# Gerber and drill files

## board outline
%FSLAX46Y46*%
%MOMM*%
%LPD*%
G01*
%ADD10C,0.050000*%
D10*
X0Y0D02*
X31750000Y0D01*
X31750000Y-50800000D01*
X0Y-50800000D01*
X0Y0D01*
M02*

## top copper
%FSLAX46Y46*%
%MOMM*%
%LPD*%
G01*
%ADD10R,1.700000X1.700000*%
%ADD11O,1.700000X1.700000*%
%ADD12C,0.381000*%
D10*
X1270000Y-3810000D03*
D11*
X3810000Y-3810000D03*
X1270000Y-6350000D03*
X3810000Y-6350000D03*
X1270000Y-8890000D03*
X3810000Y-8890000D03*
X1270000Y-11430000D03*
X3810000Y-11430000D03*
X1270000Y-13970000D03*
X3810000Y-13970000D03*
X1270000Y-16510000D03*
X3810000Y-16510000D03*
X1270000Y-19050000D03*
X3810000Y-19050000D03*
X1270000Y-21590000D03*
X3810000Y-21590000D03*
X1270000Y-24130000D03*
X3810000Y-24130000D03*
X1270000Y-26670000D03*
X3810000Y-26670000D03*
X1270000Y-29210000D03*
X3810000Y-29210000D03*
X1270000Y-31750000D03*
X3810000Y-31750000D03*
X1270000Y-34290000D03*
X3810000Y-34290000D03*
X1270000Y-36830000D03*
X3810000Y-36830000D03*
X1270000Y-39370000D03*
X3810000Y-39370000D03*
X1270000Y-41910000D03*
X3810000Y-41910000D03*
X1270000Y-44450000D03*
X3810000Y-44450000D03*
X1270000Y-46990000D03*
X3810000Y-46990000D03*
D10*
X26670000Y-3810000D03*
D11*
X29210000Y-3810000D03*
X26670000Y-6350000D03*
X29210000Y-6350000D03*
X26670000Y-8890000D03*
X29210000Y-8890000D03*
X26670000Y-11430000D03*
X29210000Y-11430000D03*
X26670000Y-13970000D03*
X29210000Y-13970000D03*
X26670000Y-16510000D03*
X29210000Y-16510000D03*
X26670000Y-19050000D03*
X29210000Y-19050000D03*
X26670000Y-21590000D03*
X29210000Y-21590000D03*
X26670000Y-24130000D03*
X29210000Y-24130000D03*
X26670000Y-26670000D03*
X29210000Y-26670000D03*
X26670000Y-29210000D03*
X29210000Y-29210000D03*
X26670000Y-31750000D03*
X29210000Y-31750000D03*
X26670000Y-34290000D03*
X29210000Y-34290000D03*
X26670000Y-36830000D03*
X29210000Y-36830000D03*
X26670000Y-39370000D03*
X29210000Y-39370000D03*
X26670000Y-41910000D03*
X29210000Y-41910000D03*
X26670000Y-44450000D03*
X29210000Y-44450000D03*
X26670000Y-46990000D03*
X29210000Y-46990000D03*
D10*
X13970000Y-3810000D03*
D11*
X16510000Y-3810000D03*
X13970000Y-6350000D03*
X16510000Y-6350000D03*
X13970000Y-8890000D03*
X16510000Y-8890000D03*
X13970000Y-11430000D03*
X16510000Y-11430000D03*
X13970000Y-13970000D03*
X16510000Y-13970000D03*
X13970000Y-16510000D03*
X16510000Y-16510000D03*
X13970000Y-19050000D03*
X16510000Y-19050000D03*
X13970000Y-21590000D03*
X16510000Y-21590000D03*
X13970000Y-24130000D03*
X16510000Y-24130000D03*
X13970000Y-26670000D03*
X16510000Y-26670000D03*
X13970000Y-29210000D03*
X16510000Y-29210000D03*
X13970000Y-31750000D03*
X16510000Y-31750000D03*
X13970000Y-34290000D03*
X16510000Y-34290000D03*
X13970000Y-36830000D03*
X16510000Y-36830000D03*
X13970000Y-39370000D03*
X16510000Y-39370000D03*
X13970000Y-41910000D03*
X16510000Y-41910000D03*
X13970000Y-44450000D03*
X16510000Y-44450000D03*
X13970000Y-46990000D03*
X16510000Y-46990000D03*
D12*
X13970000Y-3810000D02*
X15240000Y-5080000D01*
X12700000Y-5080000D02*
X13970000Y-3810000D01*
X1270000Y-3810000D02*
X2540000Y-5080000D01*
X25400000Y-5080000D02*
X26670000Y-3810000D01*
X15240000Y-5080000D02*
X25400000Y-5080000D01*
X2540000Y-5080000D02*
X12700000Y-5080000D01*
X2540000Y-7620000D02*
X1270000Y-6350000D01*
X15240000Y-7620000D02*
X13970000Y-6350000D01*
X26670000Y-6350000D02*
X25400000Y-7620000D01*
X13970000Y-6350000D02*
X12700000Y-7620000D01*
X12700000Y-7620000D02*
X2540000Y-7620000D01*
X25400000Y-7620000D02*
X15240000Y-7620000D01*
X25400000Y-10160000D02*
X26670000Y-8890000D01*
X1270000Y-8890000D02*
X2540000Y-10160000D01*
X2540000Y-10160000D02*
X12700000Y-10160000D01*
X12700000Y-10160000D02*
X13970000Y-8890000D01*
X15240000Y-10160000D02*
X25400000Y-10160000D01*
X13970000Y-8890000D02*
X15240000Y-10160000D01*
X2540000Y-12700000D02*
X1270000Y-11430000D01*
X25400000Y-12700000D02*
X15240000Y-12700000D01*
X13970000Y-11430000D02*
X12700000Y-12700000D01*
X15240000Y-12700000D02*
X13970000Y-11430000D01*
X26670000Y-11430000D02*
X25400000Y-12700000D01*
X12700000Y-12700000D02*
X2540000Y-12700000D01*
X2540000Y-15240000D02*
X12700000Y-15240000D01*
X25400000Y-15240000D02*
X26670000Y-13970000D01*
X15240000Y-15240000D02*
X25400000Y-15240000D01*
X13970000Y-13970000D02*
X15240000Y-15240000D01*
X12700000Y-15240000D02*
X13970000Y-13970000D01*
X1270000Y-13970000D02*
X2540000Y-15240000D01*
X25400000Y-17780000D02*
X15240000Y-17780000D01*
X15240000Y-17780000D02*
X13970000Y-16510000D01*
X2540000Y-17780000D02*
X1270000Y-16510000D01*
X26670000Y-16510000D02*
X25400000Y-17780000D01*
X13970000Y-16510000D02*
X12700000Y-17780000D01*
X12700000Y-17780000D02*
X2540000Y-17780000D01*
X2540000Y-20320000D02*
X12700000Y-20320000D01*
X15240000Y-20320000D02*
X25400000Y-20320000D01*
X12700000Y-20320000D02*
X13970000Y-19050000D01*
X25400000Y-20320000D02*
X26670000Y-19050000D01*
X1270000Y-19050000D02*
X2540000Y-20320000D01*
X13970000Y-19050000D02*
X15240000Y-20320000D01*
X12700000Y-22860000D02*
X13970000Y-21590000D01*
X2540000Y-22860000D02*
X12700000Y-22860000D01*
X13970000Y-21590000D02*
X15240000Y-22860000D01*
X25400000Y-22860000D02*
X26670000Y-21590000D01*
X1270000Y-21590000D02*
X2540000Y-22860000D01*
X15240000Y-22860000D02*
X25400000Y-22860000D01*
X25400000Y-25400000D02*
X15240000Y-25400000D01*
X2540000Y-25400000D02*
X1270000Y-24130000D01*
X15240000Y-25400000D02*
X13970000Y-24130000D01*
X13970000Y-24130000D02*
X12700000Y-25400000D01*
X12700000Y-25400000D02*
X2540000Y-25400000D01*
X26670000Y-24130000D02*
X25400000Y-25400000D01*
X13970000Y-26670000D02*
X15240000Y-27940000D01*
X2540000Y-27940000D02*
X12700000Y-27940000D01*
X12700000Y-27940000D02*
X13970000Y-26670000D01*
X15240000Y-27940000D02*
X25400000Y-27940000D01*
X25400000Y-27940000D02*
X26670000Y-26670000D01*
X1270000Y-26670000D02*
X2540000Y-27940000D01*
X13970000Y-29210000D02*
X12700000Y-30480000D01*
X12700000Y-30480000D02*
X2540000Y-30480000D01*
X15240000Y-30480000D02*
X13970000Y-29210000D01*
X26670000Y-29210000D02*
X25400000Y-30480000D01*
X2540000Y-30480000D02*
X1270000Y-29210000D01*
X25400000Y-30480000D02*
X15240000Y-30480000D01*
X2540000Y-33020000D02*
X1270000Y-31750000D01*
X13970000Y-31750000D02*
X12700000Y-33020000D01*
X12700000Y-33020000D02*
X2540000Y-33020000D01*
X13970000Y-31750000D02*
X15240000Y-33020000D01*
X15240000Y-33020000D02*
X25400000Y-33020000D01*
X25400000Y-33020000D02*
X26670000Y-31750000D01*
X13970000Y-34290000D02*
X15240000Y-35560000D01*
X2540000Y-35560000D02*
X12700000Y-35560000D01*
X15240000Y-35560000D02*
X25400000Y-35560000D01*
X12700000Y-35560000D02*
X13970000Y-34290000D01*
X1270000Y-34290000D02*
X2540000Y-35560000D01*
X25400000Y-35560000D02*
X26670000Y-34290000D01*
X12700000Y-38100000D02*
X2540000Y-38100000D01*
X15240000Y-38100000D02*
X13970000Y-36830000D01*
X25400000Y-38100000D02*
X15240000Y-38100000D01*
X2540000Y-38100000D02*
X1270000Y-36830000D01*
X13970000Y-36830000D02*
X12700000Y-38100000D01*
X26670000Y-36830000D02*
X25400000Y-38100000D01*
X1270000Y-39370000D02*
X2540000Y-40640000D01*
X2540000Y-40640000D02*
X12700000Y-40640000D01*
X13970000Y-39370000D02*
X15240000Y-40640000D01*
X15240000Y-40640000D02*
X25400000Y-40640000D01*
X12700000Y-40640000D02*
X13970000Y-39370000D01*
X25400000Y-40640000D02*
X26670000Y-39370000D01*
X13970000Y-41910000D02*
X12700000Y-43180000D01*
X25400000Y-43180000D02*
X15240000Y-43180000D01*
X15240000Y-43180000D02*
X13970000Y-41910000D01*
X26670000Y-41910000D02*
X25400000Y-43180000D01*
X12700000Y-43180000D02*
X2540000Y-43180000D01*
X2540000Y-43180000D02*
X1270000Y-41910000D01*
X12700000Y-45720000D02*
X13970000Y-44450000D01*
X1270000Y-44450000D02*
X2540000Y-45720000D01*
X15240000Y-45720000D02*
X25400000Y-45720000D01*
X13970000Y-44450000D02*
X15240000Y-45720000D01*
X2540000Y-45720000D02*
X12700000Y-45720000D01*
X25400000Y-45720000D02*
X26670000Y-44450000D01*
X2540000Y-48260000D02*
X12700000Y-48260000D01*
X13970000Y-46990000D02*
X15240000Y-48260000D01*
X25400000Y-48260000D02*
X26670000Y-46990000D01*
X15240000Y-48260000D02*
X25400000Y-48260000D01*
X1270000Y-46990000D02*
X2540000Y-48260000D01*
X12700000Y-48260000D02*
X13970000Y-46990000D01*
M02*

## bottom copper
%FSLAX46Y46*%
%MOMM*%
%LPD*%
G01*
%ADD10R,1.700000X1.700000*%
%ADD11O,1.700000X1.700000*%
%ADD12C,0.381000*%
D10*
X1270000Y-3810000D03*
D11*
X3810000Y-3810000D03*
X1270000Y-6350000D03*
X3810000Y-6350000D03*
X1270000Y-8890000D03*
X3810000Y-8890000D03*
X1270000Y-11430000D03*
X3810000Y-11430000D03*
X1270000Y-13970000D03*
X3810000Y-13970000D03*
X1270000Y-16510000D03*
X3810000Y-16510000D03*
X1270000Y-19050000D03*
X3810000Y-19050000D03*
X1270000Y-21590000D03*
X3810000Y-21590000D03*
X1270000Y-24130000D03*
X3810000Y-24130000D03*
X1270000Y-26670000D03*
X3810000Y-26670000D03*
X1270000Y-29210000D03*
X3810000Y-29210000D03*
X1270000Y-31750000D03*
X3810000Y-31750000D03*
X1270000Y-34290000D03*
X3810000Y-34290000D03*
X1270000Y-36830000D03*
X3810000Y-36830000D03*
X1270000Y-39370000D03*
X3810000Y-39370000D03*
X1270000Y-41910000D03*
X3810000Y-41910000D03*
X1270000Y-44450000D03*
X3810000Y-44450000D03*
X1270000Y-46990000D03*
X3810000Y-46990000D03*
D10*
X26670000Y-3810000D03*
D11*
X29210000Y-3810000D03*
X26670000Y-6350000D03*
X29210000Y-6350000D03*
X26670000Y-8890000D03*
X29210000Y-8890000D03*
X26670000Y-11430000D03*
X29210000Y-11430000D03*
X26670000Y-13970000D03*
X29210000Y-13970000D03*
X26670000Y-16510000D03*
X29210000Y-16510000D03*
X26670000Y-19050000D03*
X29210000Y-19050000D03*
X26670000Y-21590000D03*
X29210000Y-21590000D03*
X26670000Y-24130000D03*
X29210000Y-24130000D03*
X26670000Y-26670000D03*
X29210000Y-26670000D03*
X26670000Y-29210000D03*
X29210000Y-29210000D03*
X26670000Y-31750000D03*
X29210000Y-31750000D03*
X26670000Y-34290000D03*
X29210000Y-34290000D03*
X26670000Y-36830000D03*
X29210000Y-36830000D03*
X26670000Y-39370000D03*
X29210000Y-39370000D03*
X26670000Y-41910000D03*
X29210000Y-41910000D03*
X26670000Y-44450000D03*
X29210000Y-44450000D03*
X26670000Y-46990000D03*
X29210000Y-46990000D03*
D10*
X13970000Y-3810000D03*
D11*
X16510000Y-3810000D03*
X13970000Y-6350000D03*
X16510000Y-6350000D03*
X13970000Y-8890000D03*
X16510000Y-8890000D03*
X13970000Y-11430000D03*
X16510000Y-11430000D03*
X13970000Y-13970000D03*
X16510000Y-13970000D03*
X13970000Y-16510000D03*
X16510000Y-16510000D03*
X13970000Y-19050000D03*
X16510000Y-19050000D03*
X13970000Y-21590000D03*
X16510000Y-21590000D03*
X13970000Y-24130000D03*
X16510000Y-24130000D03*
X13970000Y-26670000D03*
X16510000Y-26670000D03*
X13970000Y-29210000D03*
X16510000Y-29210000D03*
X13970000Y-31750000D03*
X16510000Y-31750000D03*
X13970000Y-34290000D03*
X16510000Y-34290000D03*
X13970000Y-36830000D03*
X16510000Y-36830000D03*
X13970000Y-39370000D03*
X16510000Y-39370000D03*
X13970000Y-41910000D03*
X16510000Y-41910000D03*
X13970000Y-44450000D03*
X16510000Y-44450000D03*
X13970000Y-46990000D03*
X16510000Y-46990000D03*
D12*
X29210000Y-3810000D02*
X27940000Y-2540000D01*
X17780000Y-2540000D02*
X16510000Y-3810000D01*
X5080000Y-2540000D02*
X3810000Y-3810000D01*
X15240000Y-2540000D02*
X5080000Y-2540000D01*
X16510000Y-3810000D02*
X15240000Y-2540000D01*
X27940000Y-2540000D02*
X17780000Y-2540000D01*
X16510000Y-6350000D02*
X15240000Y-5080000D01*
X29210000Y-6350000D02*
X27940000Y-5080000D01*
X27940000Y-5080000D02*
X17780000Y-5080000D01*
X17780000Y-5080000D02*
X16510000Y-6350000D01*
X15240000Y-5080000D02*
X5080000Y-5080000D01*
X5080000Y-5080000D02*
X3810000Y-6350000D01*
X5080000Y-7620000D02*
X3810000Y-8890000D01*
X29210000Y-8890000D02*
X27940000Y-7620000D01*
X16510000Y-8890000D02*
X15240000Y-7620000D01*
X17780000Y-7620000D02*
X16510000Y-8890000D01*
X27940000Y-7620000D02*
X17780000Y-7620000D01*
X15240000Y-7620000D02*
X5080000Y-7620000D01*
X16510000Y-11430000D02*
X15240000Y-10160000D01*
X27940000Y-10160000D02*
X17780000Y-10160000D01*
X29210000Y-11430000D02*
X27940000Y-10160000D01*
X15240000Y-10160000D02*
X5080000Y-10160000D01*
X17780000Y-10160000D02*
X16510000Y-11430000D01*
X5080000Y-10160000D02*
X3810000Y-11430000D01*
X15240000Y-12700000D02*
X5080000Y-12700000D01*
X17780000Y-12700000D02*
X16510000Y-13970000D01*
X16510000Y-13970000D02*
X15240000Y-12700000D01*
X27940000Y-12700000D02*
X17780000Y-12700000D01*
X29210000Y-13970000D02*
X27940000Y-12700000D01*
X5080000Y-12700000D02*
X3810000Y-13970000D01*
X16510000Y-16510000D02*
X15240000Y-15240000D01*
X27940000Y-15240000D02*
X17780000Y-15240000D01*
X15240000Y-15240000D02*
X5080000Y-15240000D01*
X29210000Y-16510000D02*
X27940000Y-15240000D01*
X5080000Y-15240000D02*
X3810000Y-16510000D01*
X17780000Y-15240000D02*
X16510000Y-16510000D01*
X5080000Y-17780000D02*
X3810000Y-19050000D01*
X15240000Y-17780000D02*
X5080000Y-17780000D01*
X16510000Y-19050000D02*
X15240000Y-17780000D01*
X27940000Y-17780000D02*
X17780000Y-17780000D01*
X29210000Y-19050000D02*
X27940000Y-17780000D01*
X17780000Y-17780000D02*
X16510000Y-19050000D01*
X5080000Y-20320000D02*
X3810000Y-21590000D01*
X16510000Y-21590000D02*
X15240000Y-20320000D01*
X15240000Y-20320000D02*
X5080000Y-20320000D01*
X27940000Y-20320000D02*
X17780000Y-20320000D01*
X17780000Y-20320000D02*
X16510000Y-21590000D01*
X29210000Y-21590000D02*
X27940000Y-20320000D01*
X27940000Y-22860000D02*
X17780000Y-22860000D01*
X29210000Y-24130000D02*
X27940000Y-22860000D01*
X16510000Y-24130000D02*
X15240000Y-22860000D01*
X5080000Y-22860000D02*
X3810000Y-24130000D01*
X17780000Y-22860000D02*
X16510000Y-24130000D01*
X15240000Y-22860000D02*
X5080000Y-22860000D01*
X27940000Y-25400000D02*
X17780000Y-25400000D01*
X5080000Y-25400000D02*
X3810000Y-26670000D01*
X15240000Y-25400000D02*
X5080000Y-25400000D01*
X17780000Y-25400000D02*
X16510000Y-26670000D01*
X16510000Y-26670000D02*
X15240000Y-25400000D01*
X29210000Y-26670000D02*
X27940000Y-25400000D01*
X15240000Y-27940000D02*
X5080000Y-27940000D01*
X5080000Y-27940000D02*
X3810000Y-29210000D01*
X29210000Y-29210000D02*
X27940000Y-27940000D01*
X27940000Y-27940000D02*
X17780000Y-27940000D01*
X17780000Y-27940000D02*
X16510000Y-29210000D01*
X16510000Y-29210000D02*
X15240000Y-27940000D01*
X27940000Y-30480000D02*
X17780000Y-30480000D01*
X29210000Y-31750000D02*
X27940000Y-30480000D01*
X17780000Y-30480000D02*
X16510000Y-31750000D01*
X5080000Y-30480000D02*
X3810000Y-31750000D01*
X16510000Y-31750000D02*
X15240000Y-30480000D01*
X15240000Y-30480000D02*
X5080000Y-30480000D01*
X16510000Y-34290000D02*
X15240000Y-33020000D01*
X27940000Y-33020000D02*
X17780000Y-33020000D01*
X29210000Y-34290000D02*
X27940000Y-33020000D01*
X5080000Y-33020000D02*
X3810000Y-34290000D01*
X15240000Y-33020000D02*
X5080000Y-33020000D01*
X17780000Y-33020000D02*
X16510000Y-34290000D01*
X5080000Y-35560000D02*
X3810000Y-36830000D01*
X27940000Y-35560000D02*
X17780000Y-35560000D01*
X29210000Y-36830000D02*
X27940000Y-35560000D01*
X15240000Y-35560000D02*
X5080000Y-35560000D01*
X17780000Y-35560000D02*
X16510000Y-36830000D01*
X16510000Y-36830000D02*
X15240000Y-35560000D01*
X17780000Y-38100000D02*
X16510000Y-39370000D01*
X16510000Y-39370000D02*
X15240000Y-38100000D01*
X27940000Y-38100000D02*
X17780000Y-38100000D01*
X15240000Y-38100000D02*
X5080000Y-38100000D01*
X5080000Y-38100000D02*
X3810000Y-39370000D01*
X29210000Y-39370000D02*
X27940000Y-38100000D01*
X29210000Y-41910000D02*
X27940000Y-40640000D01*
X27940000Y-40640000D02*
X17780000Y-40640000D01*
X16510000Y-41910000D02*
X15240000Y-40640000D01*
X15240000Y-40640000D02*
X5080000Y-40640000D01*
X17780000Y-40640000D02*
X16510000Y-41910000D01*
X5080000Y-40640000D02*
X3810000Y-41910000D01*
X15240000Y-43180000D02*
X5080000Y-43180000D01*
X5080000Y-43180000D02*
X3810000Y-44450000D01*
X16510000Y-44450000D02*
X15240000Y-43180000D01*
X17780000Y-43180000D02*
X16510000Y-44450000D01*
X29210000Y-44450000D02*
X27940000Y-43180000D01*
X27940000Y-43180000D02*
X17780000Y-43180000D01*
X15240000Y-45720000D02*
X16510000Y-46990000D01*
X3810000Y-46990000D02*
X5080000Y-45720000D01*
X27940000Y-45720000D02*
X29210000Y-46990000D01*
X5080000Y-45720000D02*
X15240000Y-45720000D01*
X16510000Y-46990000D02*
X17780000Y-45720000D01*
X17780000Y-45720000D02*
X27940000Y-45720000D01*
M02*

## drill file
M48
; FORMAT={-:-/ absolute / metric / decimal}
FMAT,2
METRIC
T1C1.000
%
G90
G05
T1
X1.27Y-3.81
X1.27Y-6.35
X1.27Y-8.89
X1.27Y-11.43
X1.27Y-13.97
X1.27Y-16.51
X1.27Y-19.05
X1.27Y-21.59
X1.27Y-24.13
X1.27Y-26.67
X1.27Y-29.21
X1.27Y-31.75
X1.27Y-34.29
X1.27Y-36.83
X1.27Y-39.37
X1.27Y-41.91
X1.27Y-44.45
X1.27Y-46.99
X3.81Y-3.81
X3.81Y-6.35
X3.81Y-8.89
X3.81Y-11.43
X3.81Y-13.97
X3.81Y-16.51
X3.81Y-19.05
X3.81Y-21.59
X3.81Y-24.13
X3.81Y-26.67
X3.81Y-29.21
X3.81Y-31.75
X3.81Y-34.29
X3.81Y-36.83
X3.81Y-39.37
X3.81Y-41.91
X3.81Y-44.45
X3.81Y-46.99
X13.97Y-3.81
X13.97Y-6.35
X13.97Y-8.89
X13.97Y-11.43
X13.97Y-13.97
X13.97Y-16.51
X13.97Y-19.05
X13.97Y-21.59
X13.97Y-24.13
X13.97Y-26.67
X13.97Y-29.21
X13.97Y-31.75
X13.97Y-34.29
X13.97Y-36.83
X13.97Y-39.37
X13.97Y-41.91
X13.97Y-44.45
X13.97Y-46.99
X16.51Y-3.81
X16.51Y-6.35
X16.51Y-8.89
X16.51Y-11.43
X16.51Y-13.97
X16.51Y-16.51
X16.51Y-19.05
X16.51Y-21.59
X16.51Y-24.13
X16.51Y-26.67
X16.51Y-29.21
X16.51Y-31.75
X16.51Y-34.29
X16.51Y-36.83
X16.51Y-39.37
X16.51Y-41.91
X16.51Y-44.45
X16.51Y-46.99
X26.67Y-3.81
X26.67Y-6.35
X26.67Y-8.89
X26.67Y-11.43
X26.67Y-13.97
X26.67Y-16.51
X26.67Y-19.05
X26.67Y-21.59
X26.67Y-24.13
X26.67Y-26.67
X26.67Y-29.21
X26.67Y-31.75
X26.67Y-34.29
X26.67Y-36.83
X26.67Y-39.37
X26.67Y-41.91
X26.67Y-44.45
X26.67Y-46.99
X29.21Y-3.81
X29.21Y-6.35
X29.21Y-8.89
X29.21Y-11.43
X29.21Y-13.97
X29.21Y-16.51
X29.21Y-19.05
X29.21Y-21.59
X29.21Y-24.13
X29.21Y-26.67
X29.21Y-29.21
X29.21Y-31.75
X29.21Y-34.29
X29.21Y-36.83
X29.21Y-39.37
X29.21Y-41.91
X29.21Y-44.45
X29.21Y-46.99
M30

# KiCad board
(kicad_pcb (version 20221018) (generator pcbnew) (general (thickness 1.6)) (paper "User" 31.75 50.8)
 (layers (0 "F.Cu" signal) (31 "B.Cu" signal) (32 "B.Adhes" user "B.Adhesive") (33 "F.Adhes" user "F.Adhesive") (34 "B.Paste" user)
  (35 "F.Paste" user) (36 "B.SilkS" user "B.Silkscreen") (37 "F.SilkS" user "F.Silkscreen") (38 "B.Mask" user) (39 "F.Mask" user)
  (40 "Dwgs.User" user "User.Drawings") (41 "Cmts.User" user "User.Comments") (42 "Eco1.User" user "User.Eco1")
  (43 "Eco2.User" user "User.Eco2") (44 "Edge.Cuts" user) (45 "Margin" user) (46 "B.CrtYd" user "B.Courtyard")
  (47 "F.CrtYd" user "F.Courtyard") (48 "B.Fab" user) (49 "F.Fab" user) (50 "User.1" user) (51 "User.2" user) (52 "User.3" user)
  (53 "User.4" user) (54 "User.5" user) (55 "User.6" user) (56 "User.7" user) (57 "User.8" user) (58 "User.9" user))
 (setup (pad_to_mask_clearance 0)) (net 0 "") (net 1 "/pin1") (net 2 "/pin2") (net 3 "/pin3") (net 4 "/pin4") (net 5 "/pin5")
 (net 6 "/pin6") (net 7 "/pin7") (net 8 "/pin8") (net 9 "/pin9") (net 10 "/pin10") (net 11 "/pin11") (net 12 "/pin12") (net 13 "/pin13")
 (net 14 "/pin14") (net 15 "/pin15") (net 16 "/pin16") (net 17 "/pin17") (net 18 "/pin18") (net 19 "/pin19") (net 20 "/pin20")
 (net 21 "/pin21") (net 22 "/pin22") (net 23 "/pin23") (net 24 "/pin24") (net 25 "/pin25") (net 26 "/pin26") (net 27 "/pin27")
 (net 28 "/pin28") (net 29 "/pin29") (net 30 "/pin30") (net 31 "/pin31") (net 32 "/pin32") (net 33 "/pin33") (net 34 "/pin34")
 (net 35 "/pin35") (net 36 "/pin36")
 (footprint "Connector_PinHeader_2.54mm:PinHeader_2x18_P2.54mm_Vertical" (layer "F.Cu") (at 1.27 3.81)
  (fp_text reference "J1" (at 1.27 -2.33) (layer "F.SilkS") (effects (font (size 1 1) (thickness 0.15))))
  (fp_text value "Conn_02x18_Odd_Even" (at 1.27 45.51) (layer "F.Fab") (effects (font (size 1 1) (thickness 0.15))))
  (pad "1" thru_hole rect (at 0 0) (size 1.7 1.7) (drill 1) (layers "*.Cu" "*.Mask") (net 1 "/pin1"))
  (pad "2" thru_hole oval (at 2.54 0) (size 1.7 1.7) (drill 1) (layers "*.Cu" "*.Mask") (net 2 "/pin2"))
  (pad "3" thru_hole oval (at 0 2.54) (size 1.7 1.7) (drill 1) (layers "*.Cu" "*.Mask") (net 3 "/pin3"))
  (pad "4" thru_hole oval (at 2.54 2.54) (size 1.7 1.7) (drill 1) (layers "*.Cu" "*.Mask") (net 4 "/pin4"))
  (pad "5" thru_hole oval (at 0 5.08) (size 1.7 1.7) (drill 1) (layers "*.Cu" "*.Mask") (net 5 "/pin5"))
  (pad "6" thru_hole oval (at 2.54 5.08) (size 1.7 1.7) (drill 1) (layers "*.Cu" "*.Mask") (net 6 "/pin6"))
  (pad "7" thru_hole oval (at 0 7.62) (size 1.7 1.7) (drill 1) (layers "*.Cu" "*.Mask") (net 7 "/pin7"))
  (pad "8" thru_hole oval (at 2.54 7.62) (size 1.7 1.7) (drill 1) (layers "*.Cu" "*.Mask") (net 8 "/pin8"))
  (pad "9" thru_hole oval (at 0 10.16) (size 1.7 1.7) (drill 1) (layers "*.Cu" "*.Mask") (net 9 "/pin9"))
  (pad "10" thru_hole oval (at 2.54 10.16) (size 1.7 1.7) (drill 1) (layers "*.Cu" "*.Mask") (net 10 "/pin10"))
  (pad "11" thru_hole oval (at 0 12.7) (size 1.7 1.7) (drill 1) (layers "*.Cu" "*.Mask") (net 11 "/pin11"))
  (pad "12" thru_hole oval (at 2.54 12.7) (size 1.7 1.7) (drill 1) (layers "*.Cu" "*.Mask") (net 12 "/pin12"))
  (pad "13" thru_hole oval (at 0 15.24) (size 1.7 1.7) (drill 1) (layers "*.Cu" "*.Mask") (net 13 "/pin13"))
  (pad "14" thru_hole oval (at 2.54 15.24) (size 1.7 1.7) (drill 1) (layers "*.Cu" "*.Mask") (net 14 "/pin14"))
  (pad "15" thru_hole oval (at 0 17.78) (size 1.7 1.7) (drill 1) (layers "*.Cu" "*.Mask") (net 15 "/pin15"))
  (pad "16" thru_hole oval (at 2.54 17.78) (size 1.7 1.7) (drill 1) (layers "*.Cu" "*.Mask") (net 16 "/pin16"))
  (pad "17" thru_hole oval (at 0 20.32) (size 1.7 1.7) (drill 1) (layers "*.Cu" "*.Mask") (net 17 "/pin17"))
  (pad "18" thru_hole oval (at 2.54 20.32) (size 1.7 1.7) (drill 1) (layers "*.Cu" "*.Mask") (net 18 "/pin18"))
  (pad "19" thru_hole oval (at 0 22.86) (size 1.7 1.7) (drill 1) (layers "*.Cu" "*.Mask") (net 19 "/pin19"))
  (pad "20" thru_hole oval (at 2.54 22.86) (size 1.7 1.7) (drill 1) (layers "*.Cu" "*.Mask") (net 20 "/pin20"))
  (pad "21" thru_hole oval (at 0 25.4) (size 1.7 1.7) (drill 1) (layers "*.Cu" "*.Mask") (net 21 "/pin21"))
  (pad "22" thru_hole oval (at 2.54 25.4) (size 1.7 1.7) (drill 1) (layers "*.Cu" "*.Mask") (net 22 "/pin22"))
  (pad "23" thru_hole oval (at 0 27.94) (size 1.7 1.7) (drill 1) (layers "*.Cu" "*.Mask") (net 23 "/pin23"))
  (pad "24" thru_hole oval (at 2.54 27.94) (size 1.7 1.7) (drill 1) (layers "*.Cu" "*.Mask") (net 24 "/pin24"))
  (pad "25" thru_hole oval (at 0 30.48) (size 1.7 1.7) (drill 1) (layers "*.Cu" "*.Mask") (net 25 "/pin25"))
  (pad "26" thru_hole oval (at 2.54 30.48) (size 1.7 1.7) (drill 1) (layers "*.Cu" "*.Mask") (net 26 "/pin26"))
  (pad "27" thru_hole oval (at 0 33.02) (size 1.7 1.7) (drill 1) (layers "*.Cu" "*.Mask") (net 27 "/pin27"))
  (pad "28" thru_hole oval (at 2.54 33.02) (size 1.7 1.7) (drill 1) (layers "*.Cu" "*.Mask") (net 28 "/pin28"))
  (pad "29" thru_hole oval (at 0 35.56) (size 1.7 1.7) (drill 1) (layers "*.Cu" "*.Mask") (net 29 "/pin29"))
  (pad "30" thru_hole oval (at 2.54 35.56) (size 1.7 1.7) (drill 1) (layers "*.Cu" "*.Mask") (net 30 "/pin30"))
  (pad "31" thru_hole oval (at 0 38.1) (size 1.7 1.7) (drill 1) (layers "*.Cu" "*.Mask") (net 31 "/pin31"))
  (pad "32" thru_hole oval (at 2.54 38.1) (size 1.7 1.7) (drill 1) (layers "*.Cu" "*.Mask") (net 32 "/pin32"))
  (pad "33" thru_hole oval (at 0 40.64) (size 1.7 1.7) (drill 1) (layers "*.Cu" "*.Mask") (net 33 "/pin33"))
  (pad "34" thru_hole oval (at 2.54 40.64) (size 1.7 1.7) (drill 1) (layers "*.Cu" "*.Mask") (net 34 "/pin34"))
  (pad "35" thru_hole oval (at 0 43.18) (size 1.7 1.7) (drill 1) (layers "*.Cu" "*.Mask") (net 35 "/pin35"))
  (pad "36" thru_hole oval (at 2.54 43.18) (size 1.7 1.7) (drill 1) (layers "*.Cu" "*.Mask") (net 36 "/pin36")))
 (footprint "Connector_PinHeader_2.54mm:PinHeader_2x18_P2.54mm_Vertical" (layer "F.Cu") (at 26.67 3.81)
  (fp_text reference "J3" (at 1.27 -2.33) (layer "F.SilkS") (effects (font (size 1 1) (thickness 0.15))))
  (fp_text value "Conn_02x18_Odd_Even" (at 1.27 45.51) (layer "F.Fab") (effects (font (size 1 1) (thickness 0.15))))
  (pad "1" thru_hole rect (at 0 0) (size 1.7 1.7) (drill 1) (layers "*.Cu" "*.Mask") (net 1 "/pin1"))
  (pad "2" thru_hole oval (at 2.54 0) (size 1.7 1.7) (drill 1) (layers "*.Cu" "*.Mask") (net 2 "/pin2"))
  (pad "3" thru_hole oval (at 0 2.54) (size 1.7 1.7) (drill 1) (layers "*.Cu" "*.Mask") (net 3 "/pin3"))
  (pad "4" thru_hole oval (at 2.54 2.54) (size 1.7 1.7) (drill 1) (layers "*.Cu" "*.Mask") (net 4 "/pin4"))
  (pad "5" thru_hole oval (at 0 5.08) (size 1.7 1.7) (drill 1) (layers "*.Cu" "*.Mask") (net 5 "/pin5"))
  (pad "6" thru_hole oval (at 2.54 5.08) (size 1.7 1.7) (drill 1) (layers "*.Cu" "*.Mask") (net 6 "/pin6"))
  (pad "7" thru_hole oval (at 0 7.62) (size 1.7 1.7) (drill 1) (layers "*.Cu" "*.Mask") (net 7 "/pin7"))
  (pad "8" thru_hole oval (at 2.54 7.62) (size 1.7 1.7) (drill 1) (layers "*.Cu" "*.Mask") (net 8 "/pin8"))
  (pad "9" thru_hole oval (at 0 10.16) (size 1.7 1.7) (drill 1) (layers "*.Cu" "*.Mask") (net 9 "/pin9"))
  (pad "10" thru_hole oval (at 2.54 10.16) (size 1.7 1.7) (drill 1) (layers "*.Cu" "*.Mask") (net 10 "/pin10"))
  (pad "11" thru_hole oval (at 0 12.7) (size 1.7 1.7) (drill 1) (layers "*.Cu" "*.Mask") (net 11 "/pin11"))
  (pad "12" thru_hole oval (at 2.54 12.7) (size 1.7 1.7) (drill 1) (layers "*.Cu" "*.Mask") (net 12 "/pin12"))
  (pad "13" thru_hole oval (at 0 15.24) (size 1.7 1.7) (drill 1) (layers "*.Cu" "*.Mask") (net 13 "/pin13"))
  (pad "14" thru_hole oval (at 2.54 15.24) (size 1.7 1.7) (drill 1) (layers "*.Cu" "*.Mask") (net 14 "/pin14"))
  (pad "15" thru_hole oval (at 0 17.78) (size 1.7 1.7) (drill 1) (layers "*.Cu" "*.Mask") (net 15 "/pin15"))
  (pad "16" thru_hole oval (at 2.54 17.78) (size 1.7 1.7) (drill 1) (layers "*.Cu" "*.Mask") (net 16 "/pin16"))
  (pad "17" thru_hole oval (at 0 20.32) (size 1.7 1.7) (drill 1) (layers "*.Cu" "*.Mask") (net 17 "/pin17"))
  (pad "18" thru_hole oval (at 2.54 20.32) (size 1.7 1.7) (drill 1) (layers "*.Cu" "*.Mask") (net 18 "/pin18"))
  (pad "19" thru_hole oval (at 0 22.86) (size 1.7 1.7) (drill 1) (layers "*.Cu" "*.Mask") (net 19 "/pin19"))
  (pad "20" thru_hole oval (at 2.54 22.86) (size 1.7 1.7) (drill 1) (layers "*.Cu" "*.Mask") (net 20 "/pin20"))
  (pad "21" thru_hole oval (at 0 25.4) (size 1.7 1.7) (drill 1) (layers "*.Cu" "*.Mask") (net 21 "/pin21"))
  (pad "22" thru_hole oval (at 2.54 25.4) (size 1.7 1.7) (drill 1) (layers "*.Cu" "*.Mask") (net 22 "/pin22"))
  (pad "23" thru_hole oval (at 0 27.94) (size 1.7 1.7) (drill 1) (layers "*.Cu" "*.Mask") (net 23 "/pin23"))
  (pad "24" thru_hole oval (at 2.54 27.94) (size 1.7 1.7) (drill 1) (layers "*.Cu" "*.Mask") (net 24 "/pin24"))
  (pad "25" thru_hole oval (at 0 30.48) (size 1.7 1.7) (drill 1) (layers "*.Cu" "*.Mask") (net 25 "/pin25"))
  (pad "26" thru_hole oval (at 2.54 30.48) (size 1.7 1.7) (drill 1) (layers "*.Cu" "*.Mask") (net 26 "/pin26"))
  (pad "27" thru_hole oval (at 0 33.02) (size 1.7 1.7) (drill 1) (layers "*.Cu" "*.Mask") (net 27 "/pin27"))
  (pad "28" thru_hole oval (at 2.54 33.02) (size 1.7 1.7) (drill 1) (layers "*.Cu" "*.Mask") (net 28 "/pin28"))
  (pad "29" thru_hole oval (at 0 35.56) (size 1.7 1.7) (drill 1) (layers "*.Cu" "*.Mask") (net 29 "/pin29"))
  (pad "30" thru_hole oval (at 2.54 35.56) (size 1.7 1.7) (drill 1) (layers "*.Cu" "*.Mask") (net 30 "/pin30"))
  (pad "31" thru_hole oval (at 0 38.1) (size 1.7 1.7) (drill 1) (layers "*.Cu" "*.Mask") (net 31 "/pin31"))
  (pad "32" thru_hole oval (at 2.54 38.1) (size 1.7 1.7) (drill 1) (layers "*.Cu" "*.Mask") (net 32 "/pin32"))
  (pad "33" thru_hole oval (at 0 40.64) (size 1.7 1.7) (drill 1) (layers "*.Cu" "*.Mask") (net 33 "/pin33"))
  (pad "34" thru_hole oval (at 2.54 40.64) (size 1.7 1.7) (drill 1) (layers "*.Cu" "*.Mask") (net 34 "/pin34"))
  (pad "35" thru_hole oval (at 0 43.18) (size 1.7 1.7) (drill 1) (layers "*.Cu" "*.Mask") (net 35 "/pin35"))
  (pad "36" thru_hole oval (at 2.54 43.18) (size 1.7 1.7) (drill 1) (layers "*.Cu" "*.Mask") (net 36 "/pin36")))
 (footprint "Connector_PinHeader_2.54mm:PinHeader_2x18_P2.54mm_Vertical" (layer "F.Cu") (at 13.97 3.81)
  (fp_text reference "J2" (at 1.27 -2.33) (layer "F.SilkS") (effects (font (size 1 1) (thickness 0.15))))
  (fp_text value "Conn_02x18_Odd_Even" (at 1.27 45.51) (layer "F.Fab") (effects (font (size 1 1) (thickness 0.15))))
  (pad "1" thru_hole rect (at 0 0) (size 1.7 1.7) (drill 1) (layers "*.Cu" "*.Mask") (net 1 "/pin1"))
  (pad "2" thru_hole oval (at 2.54 0) (size 1.7 1.7) (drill 1) (layers "*.Cu" "*.Mask") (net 2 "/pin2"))
  (pad "3" thru_hole oval (at 0 2.54) (size 1.7 1.7) (drill 1) (layers "*.Cu" "*.Mask") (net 3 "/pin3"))
  (pad "4" thru_hole oval (at 2.54 2.54) (size 1.7 1.7) (drill 1) (layers "*.Cu" "*.Mask") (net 4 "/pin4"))
  (pad "5" thru_hole oval (at 0 5.08) (size 1.7 1.7) (drill 1) (layers "*.Cu" "*.Mask") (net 5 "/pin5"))
  (pad "6" thru_hole oval (at 2.54 5.08) (size 1.7 1.7) (drill 1) (layers "*.Cu" "*.Mask") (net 6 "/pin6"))
  (pad "7" thru_hole oval (at 0 7.62) (size 1.7 1.7) (drill 1) (layers "*.Cu" "*.Mask") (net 7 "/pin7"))
  (pad "8" thru_hole oval (at 2.54 7.62) (size 1.7 1.7) (drill 1) (layers "*.Cu" "*.Mask") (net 8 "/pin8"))
  (pad "9" thru_hole oval (at 0 10.16) (size 1.7 1.7) (drill 1) (layers "*.Cu" "*.Mask") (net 9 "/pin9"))
  (pad "10" thru_hole oval (at 2.54 10.16) (size 1.7 1.7) (drill 1) (layers "*.Cu" "*.Mask") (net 10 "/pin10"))
  (pad "11" thru_hole oval (at 0 12.7) (size 1.7 1.7) (drill 1) (layers "*.Cu" "*.Mask") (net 11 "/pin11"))
  (pad "12" thru_hole oval (at 2.54 12.7) (size 1.7 1.7) (drill 1) (layers "*.Cu" "*.Mask") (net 12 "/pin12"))
  (pad "13" thru_hole oval (at 0 15.24) (size 1.7 1.7) (drill 1) (layers "*.Cu" "*.Mask") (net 13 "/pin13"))
  (pad "14" thru_hole oval (at 2.54 15.24) (size 1.7 1.7) (drill 1) (layers "*.Cu" "*.Mask") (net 14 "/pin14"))
  (pad "15" thru_hole oval (at 0 17.78) (size 1.7 1.7) (drill 1) (layers "*.Cu" "*.Mask") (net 15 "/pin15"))
  (pad "16" thru_hole oval (at 2.54 17.78) (size 1.7 1.7) (drill 1) (layers "*.Cu" "*.Mask") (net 16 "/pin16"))
  (pad "17" thru_hole oval (at 0 20.32) (size 1.7 1.7) (drill 1) (layers "*.Cu" "*.Mask") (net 17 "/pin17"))
  (pad "18" thru_hole oval (at 2.54 20.32) (size 1.7 1.7) (drill 1) (layers "*.Cu" "*.Mask") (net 18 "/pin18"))
  (pad "19" thru_hole oval (at 0 22.86) (size 1.7 1.7) (drill 1) (layers "*.Cu" "*.Mask") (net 19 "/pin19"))
  (pad "20" thru_hole oval (at 2.54 22.86) (size 1.7 1.7) (drill 1) (layers "*.Cu" "*.Mask") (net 20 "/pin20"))
  (pad "21" thru_hole oval (at 0 25.4) (size 1.7 1.7) (drill 1) (layers "*.Cu" "*.Mask") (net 21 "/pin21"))
  (pad "22" thru_hole oval (at 2.54 25.4) (size 1.7 1.7) (drill 1) (layers "*.Cu" "*.Mask") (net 22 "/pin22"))
  (pad "23" thru_hole oval (at 0 27.94) (size 1.7 1.7) (drill 1) (layers "*.Cu" "*.Mask") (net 23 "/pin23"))
  (pad "24" thru_hole oval (at 2.54 27.94) (size 1.7 1.7) (drill 1) (layers "*.Cu" "*.Mask") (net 24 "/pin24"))
  (pad "25" thru_hole oval (at 0 30.48) (size 1.7 1.7) (drill 1) (layers "*.Cu" "*.Mask") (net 25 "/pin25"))
  (pad "26" thru_hole oval (at 2.54 30.48) (size 1.7 1.7) (drill 1) (layers "*.Cu" "*.Mask") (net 26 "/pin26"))
  (pad "27" thru_hole oval (at 0 33.02) (size 1.7 1.7) (drill 1) (layers "*.Cu" "*.Mask") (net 27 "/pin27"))
  (pad "28" thru_hole oval (at 2.54 33.02) (size 1.7 1.7) (drill 1) (layers "*.Cu" "*.Mask") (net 28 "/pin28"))
  (pad "29" thru_hole oval (at 0 35.56) (size 1.7 1.7) (drill 1) (layers "*.Cu" "*.Mask") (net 29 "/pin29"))
  (pad "30" thru_hole oval (at 2.54 35.56) (size 1.7 1.7) (drill 1) (layers "*.Cu" "*.Mask") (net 30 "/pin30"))
  (pad "31" thru_hole oval (at 0 38.1) (size 1.7 1.7) (drill 1) (layers "*.Cu" "*.Mask") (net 31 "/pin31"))
  (pad "32" thru_hole oval (at 2.54 38.1) (size 1.7 1.7) (drill 1) (layers "*.Cu" "*.Mask") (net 32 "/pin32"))
  (pad "33" thru_hole oval (at 0 40.64) (size 1.7 1.7) (drill 1) (layers "*.Cu" "*.Mask") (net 33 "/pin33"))
  (pad "34" thru_hole oval (at 2.54 40.64) (size 1.7 1.7) (drill 1) (layers "*.Cu" "*.Mask") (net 34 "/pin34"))
  (pad "35" thru_hole oval (at 0 43.18) (size 1.7 1.7) (drill 1) (layers "*.Cu" "*.Mask") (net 35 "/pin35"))
  (pad "36" thru_hole oval (at 2.54 43.18) (size 1.7 1.7) (drill 1) (layers "*.Cu" "*.Mask") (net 36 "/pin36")))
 (gr_rect (start 0 0) (end 31.75 50.8) (stroke (width 0.05) (type default)) (fill none) (layer "Edge.Cuts"))
 (segment (start 13.97 3.81) (end 15.24 5.08) (width 0.381) (layer "F.Cu") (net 1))
 (segment (start 12.7 5.08) (end 13.97 3.81) (width 0.381) (layer "F.Cu") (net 1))
 (segment (start 1.27 3.81) (end 2.54 5.08) (width 0.381) (layer "F.Cu") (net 1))
 (segment (start 25.4 5.08) (end 26.67 3.81) (width 0.381) (layer "F.Cu") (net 1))
 (segment (start 15.24 5.08) (end 25.4 5.08) (width 0.381) (layer "F.Cu") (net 1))
 (segment (start 2.54 5.08) (end 12.7 5.08) (width 0.381) (layer "F.Cu") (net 1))
 (segment (start 29.21 3.81) (end 27.94 2.54) (width 0.381) (layer "B.Cu") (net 2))
 (segment (start 17.78 2.54) (end 16.51 3.81) (width 0.381) (layer "B.Cu") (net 2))
 (segment (start 5.08 2.54) (end 3.81 3.81) (width 0.381) (layer "B.Cu") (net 2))
 (segment (start 15.24 2.54) (end 5.08 2.54) (width 0.381) (layer "B.Cu") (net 2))
 (segment (start 16.51 3.81) (end 15.24 2.54) (width 0.381) (layer "B.Cu") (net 2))
 (segment (start 27.94 2.54) (end 17.78 2.54) (width 0.381) (layer "B.Cu") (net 2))
 (segment (start 2.54 7.62) (end 1.27 6.35) (width 0.381) (layer "F.Cu") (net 3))
 (segment (start 15.24 7.62) (end 13.97 6.35) (width 0.381) (layer "F.Cu") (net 3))
 (segment (start 26.67 6.35) (end 25.4 7.62) (width 0.381) (layer "F.Cu") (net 3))
 (segment (start 13.97 6.35) (end 12.7 7.62) (width 0.381) (layer "F.Cu") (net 3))
 (segment (start 12.7 7.62) (end 2.54 7.62) (width 0.381) (layer "F.Cu") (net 3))
 (segment (start 25.4 7.62) (end 15.24 7.62) (width 0.381) (layer "F.Cu") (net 3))
 (segment (start 16.51 6.35) (end 15.24 5.08) (width 0.381) (layer "B.Cu") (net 4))
 (segment (start 29.21 6.35) (end 27.94 5.08) (width 0.381) (layer "B.Cu") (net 4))
 (segment (start 27.94 5.08) (end 17.78 5.08) (width 0.381) (layer "B.Cu") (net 4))
 (segment (start 17.78 5.08) (end 16.51 6.35) (width 0.381) (layer "B.Cu") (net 4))
 (segment (start 15.24 5.08) (end 5.08 5.08) (width 0.381) (layer "B.Cu") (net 4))
 (segment (start 5.08 5.08) (end 3.81 6.35) (width 0.381) (layer "B.Cu") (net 4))
 (segment (start 25.4 10.16) (end 26.67 8.89) (width 0.381) (layer "F.Cu") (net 5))
 (segment (start 1.27 8.89) (end 2.54 10.16) (width 0.381) (layer "F.Cu") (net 5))
 (segment (start 2.54 10.16) (end 12.7 10.16) (width 0.381) (layer "F.Cu") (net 5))
 (segment (start 12.7 10.16) (end 13.97 8.89) (width 0.381) (layer "F.Cu") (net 5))
 (segment (start 15.24 10.16) (end 25.4 10.16) (width 0.381) (layer "F.Cu") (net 5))
 (segment (start 13.97 8.89) (end 15.24 10.16) (width 0.381) (layer "F.Cu") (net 5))
 (segment (start 5.08 7.62) (end 3.81 8.89) (width 0.381) (layer "B.Cu") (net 6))
 (segment (start 29.21 8.89) (end 27.94 7.62) (width 0.381) (layer "B.Cu") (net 6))
 (segment (start 16.51 8.89) (end 15.24 7.62) (width 0.381) (layer "B.Cu") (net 6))
 (segment (start 17.78 7.62) (end 16.51 8.89) (width 0.381) (layer "B.Cu") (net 6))
 (segment (start 27.94 7.62) (end 17.78 7.62) (width 0.381) (layer "B.Cu") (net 6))
 (segment (start 15.24 7.62) (end 5.08 7.62) (width 0.381) (layer "B.Cu") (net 6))
 (segment (start 2.54 12.7) (end 1.27 11.43) (width 0.381) (layer "F.Cu") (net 7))
 (segment (start 25.4 12.7) (end 15.24 12.7) (width 0.381) (layer "F.Cu") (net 7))
 (segment (start 13.97 11.43) (end 12.7 12.7) (width 0.381) (layer "F.Cu") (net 7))
 (segment (start 15.24 12.7) (end 13.97 11.43) (width 0.381) (layer "F.Cu") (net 7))
 (segment (start 26.67 11.43) (end 25.4 12.7) (width 0.381) (layer "F.Cu") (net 7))
 (segment (start 12.7 12.7) (end 2.54 12.7) (width 0.381) (layer "F.Cu") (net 7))
 (segment (start 16.51 11.43) (end 15.24 10.16) (width 0.381) (layer "B.Cu") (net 8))
 (segment (start 27.94 10.16) (end 17.78 10.16) (width 0.381) (layer "B.Cu") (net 8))
 (segment (start 29.21 11.43) (end 27.94 10.16) (width 0.381) (layer "B.Cu") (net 8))
 (segment (start 15.24 10.16) (end 5.08 10.16) (width 0.381) (layer "B.Cu") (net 8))
 (segment (start 17.78 10.16) (end 16.51 11.43) (width 0.381) (layer "B.Cu") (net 8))
 (segment (start 5.08 10.16) (end 3.81 11.43) (width 0.381) (layer "B.Cu") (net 8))
 (segment (start 2.54 15.24) (end 12.7 15.24) (width 0.381) (layer "F.Cu") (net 9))
 (segment (start 25.4 15.24) (end 26.67 13.97) (width 0.381) (layer "F.Cu") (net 9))
 (segment (start 15.24 15.24) (end 25.4 15.24) (width 0.381) (layer "F.Cu") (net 9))
 (segment (start 13.97 13.97) (end 15.24 15.24) (width 0.381) (layer "F.Cu") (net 9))
 (segment (start 12.7 15.24) (end 13.97 13.97) (width 0.381) (layer "F.Cu") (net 9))
 (segment (start 1.27 13.97) (end 2.54 15.24) (width 0.381) (layer "F.Cu") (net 9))
 (segment (start 15.24 12.7) (end 5.08 12.7) (width 0.381) (layer "B.Cu") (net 10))
 (segment (start 17.78 12.7) (end 16.51 13.97) (width 0.381) (layer "B.Cu") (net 10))
 (segment (start 16.51 13.97) (end 15.24 12.7) (width 0.381) (layer "B.Cu") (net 10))
 (segment (start 27.94 12.7) (end 17.78 12.7) (width 0.381) (layer "B.Cu") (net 10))
 (segment (start 29.21 13.97) (end 27.94 12.7) (width 0.381) (layer "B.Cu") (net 10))
 (segment (start 5.08 12.7) (end 3.81 13.97) (width 0.381) (layer "B.Cu") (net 10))
 (segment (start 25.4 17.78) (end 15.24 17.78) (width 0.381) (layer "F.Cu") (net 11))
 (segment (start 15.24 17.78) (end 13.97 16.51) (width 0.381) (layer "F.Cu") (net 11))
 (segment (start 2.54 17.78) (end 1.27 16.51) (width 0.381) (layer "F.Cu") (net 11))
 (segment (start 26.67 16.51) (end 25.4 17.78) (width 0.381) (layer "F.Cu") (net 11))
 (segment (start 13.97 16.51) (end 12.7 17.78) (width 0.381) (layer "F.Cu") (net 11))
 (segment (start 12.7 17.78) (end 2.54 17.78) (width 0.381) (layer "F.Cu") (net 11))
 (segment (start 16.51 16.51) (end 15.24 15.24) (width 0.381) (layer "B.Cu") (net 12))
 (segment (start 27.94 15.24) (end 17.78 15.24) (width 0.381) (layer "B.Cu") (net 12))
 (segment (start 15.24 15.24) (end 5.08 15.24) (width 0.381) (layer "B.Cu") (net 12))
 (segment (start 29.21 16.51) (end 27.94 15.24) (width 0.381) (layer "B.Cu") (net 12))
 (segment (start 5.08 15.24) (end 3.81 16.51) (width 0.381) (layer "B.Cu") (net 12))
 (segment (start 17.78 15.24) (end 16.51 16.51) (width 0.381) (layer "B.Cu") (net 12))
 (segment (start 2.54 20.32) (end 12.7 20.32) (width 0.381) (layer "F.Cu") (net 13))
 (segment (start 15.24 20.32) (end 25.4 20.32) (width 0.381) (layer "F.Cu") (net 13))
 (segment (start 12.7 20.32) (end 13.97 19.05) (width 0.381) (layer "F.Cu") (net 13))
 (segment (start 25.4 20.32) (end 26.67 19.05) (width 0.381) (layer "F.Cu") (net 13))
 (segment (start 1.27 19.05) (end 2.54 20.32) (width 0.381) (layer "F.Cu") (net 13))
 (segment (start 13.97 19.05) (end 15.24 20.32) (width 0.381) (layer "F.Cu") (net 13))
 (segment (start 5.08 17.78) (end 3.81 19.05) (width 0.381) (layer "B.Cu") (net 14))
 (segment (start 15.24 17.78) (end 5.08 17.78) (width 0.381) (layer "B.Cu") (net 14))
 (segment (start 16.51 19.05) (end 15.24 17.78) (width 0.381) (layer "B.Cu") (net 14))
 (segment (start 27.94 17.78) (end 17.78 17.78) (width 0.381) (layer "B.Cu") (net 14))
 (segment (start 29.21 19.05) (end 27.94 17.78) (width 0.381) (layer "B.Cu") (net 14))
 (segment (start 17.78 17.78) (end 16.51 19.05) (width 0.381) (layer "B.Cu") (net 14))
 (segment (start 12.7 22.86) (end 13.97 21.59) (width 0.381) (layer "F.Cu") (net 15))
 (segment (start 2.54 22.86) (end 12.7 22.86) (width 0.381) (layer "F.Cu") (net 15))
 (segment (start 13.97 21.59) (end 15.24 22.86) (width 0.381) (layer "F.Cu") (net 15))
 (segment (start 25.4 22.86) (end 26.67 21.59) (width 0.381) (layer "F.Cu") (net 15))
 (segment (start 1.27 21.59) (end 2.54 22.86) (width 0.381) (layer "F.Cu") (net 15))
 (segment (start 15.24 22.86) (end 25.4 22.86) (width 0.381) (layer "F.Cu") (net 15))
 (segment (start 5.08 20.32) (end 3.81 21.59) (width 0.381) (layer "B.Cu") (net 16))
 (segment (start 16.51 21.59) (end 15.24 20.32) (width 0.381) (layer "B.Cu") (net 16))
 (segment (start 15.24 20.32) (end 5.08 20.32) (width 0.381) (layer "B.Cu") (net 16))
 (segment (start 27.94 20.32) (end 17.78 20.32) (width 0.381) (layer "B.Cu") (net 16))
 (segment (start 17.78 20.32) (end 16.51 21.59) (width 0.381) (layer "B.Cu") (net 16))
 (segment (start 29.21 21.59) (end 27.94 20.32) (width 0.381) (layer "B.Cu") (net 16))
 (segment (start 25.4 25.4) (end 15.24 25.4) (width 0.381) (layer "F.Cu") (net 17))
 (segment (start 2.54 25.4) (end 1.27 24.13) (width 0.381) (layer "F.Cu") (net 17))
 (segment (start 15.24 25.4) (end 13.97 24.13) (width 0.381) (layer "F.Cu") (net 17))
 (segment (start 13.97 24.13) (end 12.7 25.4) (width 0.381) (layer "F.Cu") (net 17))
 (segment (start 12.7 25.4) (end 2.54 25.4) (width 0.381) (layer "F.Cu") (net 17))
 (segment (start 26.67 24.13) (end 25.4 25.4) (width 0.381) (layer "F.Cu") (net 17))
 (segment (start 27.94 22.86) (end 17.78 22.86) (width 0.381) (layer "B.Cu") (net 18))
 (segment (start 29.21 24.13) (end 27.94 22.86) (width 0.381) (layer "B.Cu") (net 18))
 (segment (start 16.51 24.13) (end 15.24 22.86) (width 0.381) (layer "B.Cu") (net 18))
 (segment (start 5.08 22.86) (end 3.81 24.13) (width 0.381) (layer "B.Cu") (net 18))
 (segment (start 17.78 22.86) (end 16.51 24.13) (width 0.381) (layer "B.Cu") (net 18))
 (segment (start 15.24 22.86) (end 5.08 22.86) (width 0.381) (layer "B.Cu") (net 18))
 (segment (start 13.97 26.67) (end 15.24 27.94) (width 0.381) (layer "F.Cu") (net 19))
 (segment (start 2.54 27.94) (end 12.7 27.94) (width 0.381) (layer "F.Cu") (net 19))
 (segment (start 12.7 27.94) (end 13.97 26.67) (width 0.381) (layer "F.Cu") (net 19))
 (segment (start 15.24 27.94) (end 25.4 27.94) (width 0.381) (layer "F.Cu") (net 19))
 (segment (start 25.4 27.94) (end 26.67 26.67) (width 0.381) (layer "F.Cu") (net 19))
 (segment (start 1.27 26.67) (end 2.54 27.94) (width 0.381) (layer "F.Cu") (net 19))
 (segment (start 27.94 25.4) (end 17.78 25.4) (width 0.381) (layer "B.Cu") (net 20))
 (segment (start 5.08 25.4) (end 3.81 26.67) (width 0.381) (layer "B.Cu") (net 20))
 (segment (start 15.24 25.4) (end 5.08 25.4) (width 0.381) (layer "B.Cu") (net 20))
 (segment (start 17.78 25.4) (end 16.51 26.67) (width 0.381) (layer "B.Cu") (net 20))
 (segment (start 16.51 26.67) (end 15.24 25.4) (width 0.381) (layer "B.Cu") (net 20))
 (segment (start 29.21 26.67) (end 27.94 25.4) (width 0.381) (layer "B.Cu") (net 20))
 (segment (start 13.97 29.21) (end 12.7 30.48) (width 0.381) (layer "F.Cu") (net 21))
 (segment (start 12.7 30.48) (end 2.54 30.48) (width 0.381) (layer "F.Cu") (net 21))
 (segment (start 15.24 30.48) (end 13.97 29.21) (width 0.381) (layer "F.Cu") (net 21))
 (segment (start 26.67 29.21) (end 25.4 30.48) (width 0.381) (layer "F.Cu") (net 21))
 (segment (start 2.54 30.48) (end 1.27 29.21) (width 0.381) (layer "F.Cu") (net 21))
 (segment (start 25.4 30.48) (end 15.24 30.48) (width 0.381) (layer "F.Cu") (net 21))
 (segment (start 15.24 27.94) (end 5.08 27.94) (width 0.381) (layer "B.Cu") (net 22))
 (segment (start 5.08 27.94) (end 3.81 29.21) (width 0.381) (layer "B.Cu") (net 22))
 (segment (start 29.21 29.21) (end 27.94 27.94) (width 0.381) (layer "B.Cu") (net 22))
 (segment (start 27.94 27.94) (end 17.78 27.94) (width 0.381) (layer "B.Cu") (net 22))
 (segment (start 17.78 27.94) (end 16.51 29.21) (width 0.381) (layer "B.Cu") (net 22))
 (segment (start 16.51 29.21) (end 15.24 27.94) (width 0.381) (layer "B.Cu") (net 22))
 (segment (start 2.54 33.02) (end 1.27 31.75) (width 0.381) (layer "F.Cu") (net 23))
 (segment (start 13.97 31.75) (end 12.7 33.02) (width 0.381) (layer "F.Cu") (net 23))
 (segment (start 12.7 33.02) (end 2.54 33.02) (width 0.381) (layer "F.Cu") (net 23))
 (segment (start 13.97 31.75) (end 15.24 33.02) (width 0.381) (layer "F.Cu") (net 23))
 (segment (start 15.24 33.02) (end 25.4 33.02) (width 0.381) (layer "F.Cu") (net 23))
 (segment (start 25.4 33.02) (end 26.67 31.75) (width 0.381) (layer "F.Cu") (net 23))
 (segment (start 27.94 30.48) (end 17.78 30.48) (width 0.381) (layer "B.Cu") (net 24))
 (segment (start 29.21 31.75) (end 27.94 30.48) (width 0.381) (layer "B.Cu") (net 24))
 (segment (start 17.78 30.48) (end 16.51 31.75) (width 0.381) (layer "B.Cu") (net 24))
 (segment (start 5.08 30.48) (end 3.81 31.75) (width 0.381) (layer "B.Cu") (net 24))
 (segment (start 16.51 31.75) (end 15.24 30.48) (width 0.381) (layer "B.Cu") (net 24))
 (segment (start 15.24 30.48) (end 5.08 30.48) (width 0.381) (layer "B.Cu") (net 24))
 (segment (start 13.97 34.29) (end 15.24 35.56) (width 0.381) (layer "F.Cu") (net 25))
 (segment (start 2.54 35.56) (end 12.7 35.56) (width 0.381) (layer "F.Cu") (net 25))
 (segment (start 15.24 35.56) (end 25.4 35.56) (width 0.381) (layer "F.Cu") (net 25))
 (segment (start 12.7 35.56) (end 13.97 34.29) (width 0.381) (layer "F.Cu") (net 25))
 (segment (start 1.27 34.29) (end 2.54 35.56) (width 0.381) (layer "F.Cu") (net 25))
 (segment (start 25.4 35.56) (end 26.67 34.29) (width 0.381) (layer "F.Cu") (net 25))
 (segment (start 16.51 34.29) (end 15.24 33.02) (width 0.381) (layer "B.Cu") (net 26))
 (segment (start 27.94 33.02) (end 17.78 33.02) (width 0.381) (layer "B.Cu") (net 26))
 (segment (start 29.21 34.29) (end 27.94 33.02) (width 0.381) (layer "B.Cu") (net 26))
 (segment (start 5.08 33.02) (end 3.81 34.29) (width 0.381) (layer "B.Cu") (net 26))
 (segment (start 15.24 33.02) (end 5.08 33.02) (width 0.381) (layer "B.Cu") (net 26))
 (segment (start 17.78 33.02) (end 16.51 34.29) (width 0.381) (layer "B.Cu") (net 26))
 (segment (start 12.7 38.1) (end 2.54 38.1) (width 0.381) (layer "F.Cu") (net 27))
 (segment (start 15.24 38.1) (end 13.97 36.83) (width 0.381) (layer "F.Cu") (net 27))
 (segment (start 25.4 38.1) (end 15.24 38.1) (width 0.381) (layer "F.Cu") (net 27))
 (segment (start 2.54 38.1) (end 1.27 36.83) (width 0.381) (layer "F.Cu") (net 27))
 (segment (start 13.97 36.83) (end 12.7 38.1) (width 0.381) (layer "F.Cu") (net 27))
 (segment (start 26.67 36.83) (end 25.4 38.1) (width 0.381) (layer "F.Cu") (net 27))
 (segment (start 5.08 35.56) (end 3.81 36.83) (width 0.381) (layer "B.Cu") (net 28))
 (segment (start 27.94 35.56) (end 17.78 35.56) (width 0.381) (layer "B.Cu") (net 28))
 (segment (start 29.21 36.83) (end 27.94 35.56) (width 0.381) (layer "B.Cu") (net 28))
 (segment (start 15.24 35.56) (end 5.08 35.56) (width 0.381) (layer "B.Cu") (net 28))
 (segment (start 17.78 35.56) (end 16.51 36.83) (width 0.381) (layer "B.Cu") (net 28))
 (segment (start 16.51 36.83) (end 15.24 35.56) (width 0.381) (layer "B.Cu") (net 28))
 (segment (start 1.27 39.37) (end 2.54 40.64) (width 0.381) (layer "F.Cu") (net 29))
 (segment (start 2.54 40.64) (end 12.7 40.64) (width 0.381) (layer "F.Cu") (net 29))
 (segment (start 13.97 39.37) (end 15.24 40.64) (width 0.381) (layer "F.Cu") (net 29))
 (segment (start 15.24 40.64) (end 25.4 40.64) (width 0.381) (layer "F.Cu") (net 29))
 (segment (start 12.7 40.64) (end 13.97 39.37) (width 0.381) (layer "F.Cu") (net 29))
 (segment (start 25.4 40.64) (end 26.67 39.37) (width 0.381) (layer "F.Cu") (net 29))
 (segment (start 17.78 38.1) (end 16.51 39.37) (width 0.381) (layer "B.Cu") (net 30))
 (segment (start 16.51 39.37) (end 15.24 38.1) (width 0.381) (layer "B.Cu") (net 30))
 (segment (start 27.94 38.1) (end 17.78 38.1) (width 0.381) (layer "B.Cu") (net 30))
 (segment (start 15.24 38.1) (end 5.08 38.1) (width 0.381) (layer "B.Cu") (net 30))
 (segment (start 5.08 38.1) (end 3.81 39.37) (width 0.381) (layer "B.Cu") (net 30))
 (segment (start 29.21 39.37) (end 27.94 38.1) (width 0.381) (layer "B.Cu") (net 30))
 (segment (start 13.97 41.91) (end 12.7 43.18) (width 0.381) (layer "F.Cu") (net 31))
 (segment (start 25.4 43.18) (end 15.24 43.18) (width 0.381) (layer "F.Cu") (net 31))
 (segment (start 15.24 43.18) (end 13.97 41.91) (width 0.381) (layer "F.Cu") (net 31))
 (segment (start 26.67 41.91) (end 25.4 43.18) (width 0.381) (layer "F.Cu") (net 31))
 (segment (start 12.7 43.18) (end 2.54 43.18) (width 0.381) (layer "F.Cu") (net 31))
 (segment (start 2.54 43.18) (end 1.27 41.91) (width 0.381) (layer "F.Cu") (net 31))
 (segment (start 29.21 41.91) (end 27.94 40.64) (width 0.381) (layer "B.Cu") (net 32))
 (segment (start 27.94 40.64) (end 17.78 40.64) (width 0.381) (layer "B.Cu") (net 32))
 (segment (start 16.51 41.91) (end 15.24 40.64) (width 0.381) (layer "B.Cu") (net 32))
 (segment (start 15.24 40.64) (end 5.08 40.64) (width 0.381) (layer "B.Cu") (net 32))
 (segment (start 17.78 40.64) (end 16.51 41.91) (width 0.381) (layer "B.Cu") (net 32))
 (segment (start 5.08 40.64) (end 3.81 41.91) (width 0.381) (layer "B.Cu") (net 32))
 (segment (start 12.7 45.72) (end 13.97 44.45) (width 0.381) (layer "F.Cu") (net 33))
 (segment (start 1.27 44.45) (end 2.54 45.72) (width 0.381) (layer "F.Cu") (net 33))
 (segment (start 15.24 45.72) (end 25.4 45.72) (width 0.381) (layer "F.Cu") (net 33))
 (segment (start 13.97 44.45) (end 15.24 45.72) (width 0.381) (layer "F.Cu") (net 33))
 (segment (start 2.54 45.72) (end 12.7 45.72) (width 0.381) (layer "F.Cu") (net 33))
 (segment (start 25.4 45.72) (end 26.67 44.45) (width 0.381) (layer "F.Cu") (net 33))
 (segment (start 15.24 43.18) (end 5.08 43.18) (width 0.381) (layer "B.Cu") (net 34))
 (segment (start 5.08 43.18) (end 3.81 44.45) (width 0.381) (layer "B.Cu") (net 34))
 (segment (start 16.51 44.45) (end 15.24 43.18) (width 0.381) (layer "B.Cu") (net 34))
 (segment (start 17.78 43.18) (end 16.51 44.45) (width 0.381) (layer "B.Cu") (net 34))
 (segment (start 29.21 44.45) (end 27.94 43.18) (width 0.381) (layer "B.Cu") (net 34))
 (segment (start 27.94 43.18) (end 17.78 43.18) (width 0.381) (layer "B.Cu") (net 34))
 (segment (start 2.54 48.26) (end 12.7 48.26) (width 0.381) (layer "F.Cu") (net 35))
 (segment (start 13.97 46.99) (end 15.24 48.26) (width 0.381) (layer "F.Cu") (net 35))
 (segment (start 25.4 48.26) (end 26.67 46.99) (width 0.381) (layer "F.Cu") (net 35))
 (segment (start 15.24 48.26) (end 25.4 48.26) (width 0.381) (layer "F.Cu") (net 35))
 (segment (start 1.27 46.99) (end 2.54 48.26) (width 0.381) (layer "F.Cu") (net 35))
 (segment (start 12.7 48.26) (end 13.97 46.99) (width 0.381) (layer "F.Cu") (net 35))
 (segment (start 15.24 45.72) (end 16.51 46.99) (width 0.381) (layer "B.Cu") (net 36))
 (segment (start 3.81 46.99) (end 5.08 45.72) (width 0.381) (layer "B.Cu") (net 36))
 (segment (start 27.94 45.72) (end 29.21 46.99) (width 0.381) (layer "B.Cu") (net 36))
 (segment (start 5.08 45.72) (end 15.24 45.72) (width 0.381) (layer "B.Cu") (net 36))
 (segment (start 16.51 46.99) (end 17.78 45.72) (width 0.381) (layer "B.Cu") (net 36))
 (segment (start 17.78 45.72) (end 27.94 45.72) (width 0.381) (layer "B.Cu") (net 36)))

